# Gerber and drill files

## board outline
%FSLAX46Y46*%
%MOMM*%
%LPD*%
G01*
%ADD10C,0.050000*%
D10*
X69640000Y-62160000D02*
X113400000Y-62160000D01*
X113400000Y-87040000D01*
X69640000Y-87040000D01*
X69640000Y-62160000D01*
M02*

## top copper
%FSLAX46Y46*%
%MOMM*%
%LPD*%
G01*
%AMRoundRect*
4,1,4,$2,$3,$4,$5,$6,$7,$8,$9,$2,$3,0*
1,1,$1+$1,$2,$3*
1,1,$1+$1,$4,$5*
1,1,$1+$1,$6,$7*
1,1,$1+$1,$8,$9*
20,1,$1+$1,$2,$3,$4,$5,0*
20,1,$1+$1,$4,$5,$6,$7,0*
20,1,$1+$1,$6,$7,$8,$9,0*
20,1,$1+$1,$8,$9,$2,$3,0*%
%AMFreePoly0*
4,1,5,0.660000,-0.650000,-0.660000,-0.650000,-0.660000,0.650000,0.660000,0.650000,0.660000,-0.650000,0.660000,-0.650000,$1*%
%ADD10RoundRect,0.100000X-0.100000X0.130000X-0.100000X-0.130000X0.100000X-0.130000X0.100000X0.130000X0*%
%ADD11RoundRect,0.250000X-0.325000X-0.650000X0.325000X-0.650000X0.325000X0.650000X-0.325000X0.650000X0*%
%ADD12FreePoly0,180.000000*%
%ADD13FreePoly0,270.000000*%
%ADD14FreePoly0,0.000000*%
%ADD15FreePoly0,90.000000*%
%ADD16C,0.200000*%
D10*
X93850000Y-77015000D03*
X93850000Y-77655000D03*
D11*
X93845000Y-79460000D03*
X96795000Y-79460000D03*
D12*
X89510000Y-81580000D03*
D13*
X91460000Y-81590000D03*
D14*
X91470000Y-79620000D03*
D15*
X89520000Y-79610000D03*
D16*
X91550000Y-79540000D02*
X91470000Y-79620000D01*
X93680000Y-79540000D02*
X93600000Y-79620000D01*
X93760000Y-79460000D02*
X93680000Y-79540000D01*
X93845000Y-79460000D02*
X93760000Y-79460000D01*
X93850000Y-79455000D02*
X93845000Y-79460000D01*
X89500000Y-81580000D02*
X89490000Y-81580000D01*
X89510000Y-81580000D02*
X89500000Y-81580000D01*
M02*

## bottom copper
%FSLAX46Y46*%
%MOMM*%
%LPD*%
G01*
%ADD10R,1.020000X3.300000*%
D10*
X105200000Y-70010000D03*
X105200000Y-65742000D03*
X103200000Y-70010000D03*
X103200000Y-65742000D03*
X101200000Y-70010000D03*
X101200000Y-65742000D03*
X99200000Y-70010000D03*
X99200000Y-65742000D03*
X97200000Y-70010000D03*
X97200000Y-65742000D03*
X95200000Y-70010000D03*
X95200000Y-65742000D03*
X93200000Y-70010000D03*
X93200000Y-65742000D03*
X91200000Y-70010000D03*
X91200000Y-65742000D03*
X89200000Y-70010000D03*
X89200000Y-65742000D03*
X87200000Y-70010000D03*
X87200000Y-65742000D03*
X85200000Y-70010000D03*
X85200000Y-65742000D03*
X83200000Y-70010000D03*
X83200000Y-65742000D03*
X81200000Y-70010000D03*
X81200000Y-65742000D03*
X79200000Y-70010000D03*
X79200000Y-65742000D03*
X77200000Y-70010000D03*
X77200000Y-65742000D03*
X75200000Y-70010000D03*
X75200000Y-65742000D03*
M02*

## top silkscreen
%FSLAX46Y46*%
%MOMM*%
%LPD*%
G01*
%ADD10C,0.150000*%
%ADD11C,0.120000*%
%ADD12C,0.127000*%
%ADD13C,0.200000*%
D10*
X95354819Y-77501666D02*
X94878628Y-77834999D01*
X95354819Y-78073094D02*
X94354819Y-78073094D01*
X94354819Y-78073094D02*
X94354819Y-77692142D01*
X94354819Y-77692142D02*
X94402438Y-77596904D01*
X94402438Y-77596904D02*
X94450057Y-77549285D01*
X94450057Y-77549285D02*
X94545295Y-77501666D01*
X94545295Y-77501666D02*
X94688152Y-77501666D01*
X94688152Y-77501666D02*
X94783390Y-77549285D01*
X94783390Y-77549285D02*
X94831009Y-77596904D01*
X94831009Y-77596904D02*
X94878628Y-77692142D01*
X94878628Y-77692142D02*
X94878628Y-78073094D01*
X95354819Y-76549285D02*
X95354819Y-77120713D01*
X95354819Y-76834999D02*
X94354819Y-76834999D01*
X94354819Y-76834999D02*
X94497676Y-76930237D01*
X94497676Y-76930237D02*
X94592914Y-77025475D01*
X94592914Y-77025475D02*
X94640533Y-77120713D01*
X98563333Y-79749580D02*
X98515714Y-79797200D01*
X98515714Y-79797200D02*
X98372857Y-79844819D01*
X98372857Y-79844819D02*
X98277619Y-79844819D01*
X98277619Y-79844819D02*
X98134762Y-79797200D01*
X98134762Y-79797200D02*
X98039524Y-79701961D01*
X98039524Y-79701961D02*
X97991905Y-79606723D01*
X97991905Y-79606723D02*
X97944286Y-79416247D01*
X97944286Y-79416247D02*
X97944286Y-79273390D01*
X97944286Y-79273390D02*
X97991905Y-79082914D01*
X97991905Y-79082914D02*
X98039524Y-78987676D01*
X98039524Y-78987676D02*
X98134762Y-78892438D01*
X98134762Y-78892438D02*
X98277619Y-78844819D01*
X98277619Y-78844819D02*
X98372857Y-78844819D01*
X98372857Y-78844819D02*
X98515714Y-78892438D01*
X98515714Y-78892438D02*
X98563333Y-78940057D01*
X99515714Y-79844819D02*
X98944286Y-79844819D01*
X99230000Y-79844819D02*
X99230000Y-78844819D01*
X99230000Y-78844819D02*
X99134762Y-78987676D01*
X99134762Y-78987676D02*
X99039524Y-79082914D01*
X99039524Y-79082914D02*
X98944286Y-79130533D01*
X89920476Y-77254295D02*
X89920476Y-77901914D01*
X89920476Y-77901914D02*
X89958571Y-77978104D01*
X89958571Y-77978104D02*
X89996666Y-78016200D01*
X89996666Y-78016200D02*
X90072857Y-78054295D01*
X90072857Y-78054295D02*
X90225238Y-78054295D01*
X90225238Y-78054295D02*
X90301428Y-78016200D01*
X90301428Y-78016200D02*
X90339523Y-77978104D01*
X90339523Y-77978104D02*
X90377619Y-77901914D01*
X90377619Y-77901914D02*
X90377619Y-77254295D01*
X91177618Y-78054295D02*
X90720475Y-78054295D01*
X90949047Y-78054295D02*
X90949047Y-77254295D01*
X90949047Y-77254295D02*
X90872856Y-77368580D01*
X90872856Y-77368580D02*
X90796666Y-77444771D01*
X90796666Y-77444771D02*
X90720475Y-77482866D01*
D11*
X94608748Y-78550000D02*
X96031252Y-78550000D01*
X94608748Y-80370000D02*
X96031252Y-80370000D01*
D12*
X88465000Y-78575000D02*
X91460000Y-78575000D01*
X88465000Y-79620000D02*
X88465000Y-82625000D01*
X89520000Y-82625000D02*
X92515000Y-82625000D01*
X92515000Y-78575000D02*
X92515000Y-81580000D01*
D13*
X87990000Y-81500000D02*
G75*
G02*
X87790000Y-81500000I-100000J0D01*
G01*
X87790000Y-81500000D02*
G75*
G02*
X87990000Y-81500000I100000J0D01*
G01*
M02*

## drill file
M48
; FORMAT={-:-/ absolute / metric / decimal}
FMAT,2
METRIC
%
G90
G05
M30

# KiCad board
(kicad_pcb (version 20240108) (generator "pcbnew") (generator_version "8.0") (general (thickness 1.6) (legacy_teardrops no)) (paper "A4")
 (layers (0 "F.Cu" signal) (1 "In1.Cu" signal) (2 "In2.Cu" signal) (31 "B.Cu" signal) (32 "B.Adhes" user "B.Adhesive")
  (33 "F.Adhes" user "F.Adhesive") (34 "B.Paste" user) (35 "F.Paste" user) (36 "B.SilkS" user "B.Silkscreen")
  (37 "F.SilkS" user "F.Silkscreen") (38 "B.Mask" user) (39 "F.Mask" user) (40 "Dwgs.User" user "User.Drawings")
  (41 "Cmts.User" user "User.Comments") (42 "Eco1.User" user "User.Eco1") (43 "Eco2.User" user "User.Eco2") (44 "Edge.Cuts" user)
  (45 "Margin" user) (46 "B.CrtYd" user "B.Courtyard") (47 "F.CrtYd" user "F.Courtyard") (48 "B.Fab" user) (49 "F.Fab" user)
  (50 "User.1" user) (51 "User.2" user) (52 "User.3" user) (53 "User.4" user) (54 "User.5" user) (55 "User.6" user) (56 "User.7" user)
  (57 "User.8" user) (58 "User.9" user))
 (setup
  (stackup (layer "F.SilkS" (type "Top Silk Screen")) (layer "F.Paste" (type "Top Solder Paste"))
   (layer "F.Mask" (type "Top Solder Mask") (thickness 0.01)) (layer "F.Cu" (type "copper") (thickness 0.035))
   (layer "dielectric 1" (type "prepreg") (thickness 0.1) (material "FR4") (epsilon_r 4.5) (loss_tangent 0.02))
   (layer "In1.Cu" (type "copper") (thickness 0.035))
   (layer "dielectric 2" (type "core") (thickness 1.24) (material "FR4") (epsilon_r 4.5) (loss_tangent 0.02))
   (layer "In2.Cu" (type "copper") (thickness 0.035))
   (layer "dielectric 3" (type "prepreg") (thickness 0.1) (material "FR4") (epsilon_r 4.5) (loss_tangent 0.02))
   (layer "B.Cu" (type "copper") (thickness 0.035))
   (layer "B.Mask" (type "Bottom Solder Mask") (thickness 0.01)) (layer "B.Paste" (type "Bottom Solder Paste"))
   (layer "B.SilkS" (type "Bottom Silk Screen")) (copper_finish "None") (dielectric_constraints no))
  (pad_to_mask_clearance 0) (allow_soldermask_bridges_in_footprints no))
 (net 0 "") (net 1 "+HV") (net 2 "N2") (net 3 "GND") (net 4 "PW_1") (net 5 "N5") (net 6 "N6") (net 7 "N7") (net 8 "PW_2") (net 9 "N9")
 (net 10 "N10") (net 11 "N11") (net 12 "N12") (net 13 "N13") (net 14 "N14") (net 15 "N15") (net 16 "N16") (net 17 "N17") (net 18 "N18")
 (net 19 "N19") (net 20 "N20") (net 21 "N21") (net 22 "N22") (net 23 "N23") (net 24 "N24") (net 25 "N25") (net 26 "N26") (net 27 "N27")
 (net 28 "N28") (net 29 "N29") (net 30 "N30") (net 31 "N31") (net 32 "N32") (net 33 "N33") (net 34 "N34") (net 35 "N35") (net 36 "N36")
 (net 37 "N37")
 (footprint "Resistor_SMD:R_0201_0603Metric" (layer "F.Cu") (at 93.85 77.335 -90)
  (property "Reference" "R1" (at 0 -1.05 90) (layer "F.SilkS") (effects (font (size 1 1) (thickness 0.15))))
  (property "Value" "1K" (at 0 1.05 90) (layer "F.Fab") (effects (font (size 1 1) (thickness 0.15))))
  (pad "" smd roundrect (at -0.345 0 270) (size 0.318 0.36) (layers "F.Paste") (roundrect_rratio 0.25))
  (pad "" smd roundrect (at 0.345 0 270) (size 0.318 0.36) (layers "F.Paste") (roundrect_rratio 0.25))
  (pad "1" smd roundrect (at -0.32 0 270) (size 0.46 0.4) (layers "F.Cu" "F.Mask") (roundrect_rratio 0.25) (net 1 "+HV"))
  (pad "2" smd roundrect (at 0.32 0 270) (size 0.46 0.4) (layers "F.Cu" "F.Mask") (roundrect_rratio 0.25) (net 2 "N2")))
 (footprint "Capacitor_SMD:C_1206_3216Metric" (layer "F.Cu") (at 95.32 79.46)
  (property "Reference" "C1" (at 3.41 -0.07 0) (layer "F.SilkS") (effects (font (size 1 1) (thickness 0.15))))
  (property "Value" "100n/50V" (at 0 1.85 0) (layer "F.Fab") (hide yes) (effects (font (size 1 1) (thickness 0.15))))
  (fp_line (start -0.711252 -0.91) (end 0.711252 -0.91) (stroke (width 0.12) (type solid)) (layer "F.SilkS"))
  (fp_line (start -0.711252 0.91) (end 0.711252 0.91) (stroke (width 0.12) (type solid)) (layer "F.SilkS"))
  (pad "1" smd roundrect (at -1.475 0) (size 1.15 1.8) (layers "F.Cu" "F.Paste" "F.Mask") (roundrect_rratio 0.217391) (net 2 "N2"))
  (pad "2" smd roundrect (at 1.475 0) (size 1.15 1.8) (layers "F.Cu" "F.Paste" "F.Mask") (roundrect_rratio 0.217391) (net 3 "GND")))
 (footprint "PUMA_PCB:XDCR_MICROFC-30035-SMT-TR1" (layer "F.Cu") (at 90.49 80.6)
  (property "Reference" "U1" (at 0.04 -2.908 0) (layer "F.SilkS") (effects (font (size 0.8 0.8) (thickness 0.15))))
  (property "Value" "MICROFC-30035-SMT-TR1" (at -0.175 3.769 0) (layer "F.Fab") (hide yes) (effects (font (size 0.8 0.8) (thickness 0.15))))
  (fp_line (start -2.025 -2.025) (end 0.97 -2.025) (stroke (width 0.127) (type solid)) (layer "F.SilkS"))
  (fp_line (start -2.025 -0.98) (end -2.025 2.025) (stroke (width 0.127) (type solid)) (layer "F.SilkS"))
  (fp_line (start -0.97 2.025) (end 2.025 2.025) (stroke (width 0.127) (type solid)) (layer "F.SilkS"))
  (fp_line (start 2.025 -2.025) (end 2.025 0.98) (stroke (width 0.127) (type solid)) (layer "F.SilkS"))
  (fp_circle (center -2.6 0.9) (end -2.5 0.9) (stroke (width 0.2) (type solid)) (fill none) (layer "F.SilkS"))
  (pad "1" smd custom (at -0.98 0.98 180) (size 1.32 1.3) (layers "F.Cu") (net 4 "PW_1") (options (clearance outline) (anchor rect))
   (primitives))
  (pad "2" smd custom (at 0.97 0.99 270) (size 1.32 1.3) (layers "F.Cu") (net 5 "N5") (options (clearance outline) (anchor rect))
   (primitives))
  (pad "3" smd custom (at 0.98 -0.98) (size 1.32 1.3) (layers "F.Cu") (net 2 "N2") (options (clearance outline) (anchor rect)) (primitives)
   (teardrops (best_length_ratio 0.5) (max_length 1) (best_width_ratio 1) (max_width 2) (curve_points 5) (filter_ratio 0.9) (enabled yes)
    (allow_two_segments yes) (prefer_zone_connections yes)))
  (pad "4" smd custom (at -0.97 -0.99 90) (size 1.32 1.3) (layers "F.Cu") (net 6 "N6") (options (clearance outline) (anchor rect))
   (primitives)))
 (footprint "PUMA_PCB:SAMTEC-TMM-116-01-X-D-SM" (layer "B.Cu") (at 90.2 67.876 180)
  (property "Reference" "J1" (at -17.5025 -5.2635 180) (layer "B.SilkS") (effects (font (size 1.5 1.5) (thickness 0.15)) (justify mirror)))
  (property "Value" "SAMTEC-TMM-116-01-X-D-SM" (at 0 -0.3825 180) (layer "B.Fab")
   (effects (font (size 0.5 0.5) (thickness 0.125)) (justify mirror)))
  (pad "1" smd rect (at -15 -2.134 180) (size 1.02 3.3) (layers "B.Cu" "B.Paste") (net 4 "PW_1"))
  (pad "2" smd rect (at -15 2.134 180) (size 1.02 3.3) (layers "B.Cu" "B.Paste") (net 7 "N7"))
  (pad "3" smd rect (at -13 -2.134 180) (size 1.02 3.3) (layers "B.Cu" "B.Paste") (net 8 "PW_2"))
  (pad "4" smd rect (at -13 2.134 180) (size 1.02 3.3) (layers "B.Cu" "B.Paste") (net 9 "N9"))
  (pad "5" smd rect (at -11 -2.134 180) (size 1.02 3.3) (layers "B.Cu" "B.Paste") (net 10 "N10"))
  (pad "6" smd rect (at -11 2.134 180) (size 1.02 3.3) (layers "B.Cu" "B.Paste") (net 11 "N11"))
  (pad "7" smd rect (at -9 -2.134 180) (size 1.02 3.3) (layers "B.Cu" "B.Paste") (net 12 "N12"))
  (pad "8" smd rect (at -9 2.134 180) (size 1.02 3.3) (layers "B.Cu" "B.Paste") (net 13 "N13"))
  (pad "9" smd rect (at -7 -2.134 180) (size 1.02 3.3) (layers "B.Cu" "B.Paste") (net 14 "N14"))
  (pad "10" smd rect (at -7 2.134 180) (size 1.02 3.3) (layers "B.Cu" "B.Paste") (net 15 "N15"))
  (pad "11" smd rect (at -5 -2.134 180) (size 1.02 3.3) (layers "B.Cu" "B.Paste") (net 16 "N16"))
  (pad "12" smd rect (at -5 2.134 180) (size 1.02 3.3) (layers "B.Cu" "B.Paste") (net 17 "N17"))
  (pad "13" smd rect (at -3 -2.134 180) (size 1.02 3.3) (layers "B.Cu" "B.Paste") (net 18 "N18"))
  (pad "14" smd rect (at -3 2.134 180) (size 1.02 3.3) (layers "B.Cu" "B.Paste") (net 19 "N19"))
  (pad "15" smd rect (at -1 -2.134 180) (size 1.02 3.3) (layers "B.Cu" "B.Paste") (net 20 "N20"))
  (pad "16" smd rect (at -1 2.134 180) (size 1.02 3.3) (layers "B.Cu" "B.Paste") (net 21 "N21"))
  (pad "17" smd rect (at 1 -2.134 180) (size 1.02 3.3) (layers "B.Cu" "B.Paste") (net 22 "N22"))
  (pad "18" smd rect (at 1 2.134 180) (size 1.02 3.3) (layers "B.Cu" "B.Paste") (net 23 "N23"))
  (pad "19" smd rect (at 3 -2.134 180) (size 1.02 3.3) (layers "B.Cu" "B.Paste") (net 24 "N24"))
  (pad "20" smd rect (at 3 2.134 180) (size 1.02 3.3) (layers "B.Cu" "B.Paste") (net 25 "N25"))
  (pad "21" smd rect (at 5 -2.134 180) (size 1.02 3.3) (layers "B.Cu" "B.Paste") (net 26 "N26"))
  (pad "22" smd rect (at 5 2.134 180) (size 1.02 3.3) (layers "B.Cu" "B.Paste") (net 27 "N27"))
  (pad "23" smd rect (at 7 -2.134 180) (size 1.02 3.3) (layers "B.Cu" "B.Paste") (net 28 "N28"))
  (pad "24" smd rect (at 7 2.134 180) (size 1.02 3.3) (layers "B.Cu" "B.Paste") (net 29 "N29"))
  (pad "25" smd rect (at 9 -2.134 180) (size 1.02 3.3) (layers "B.Cu" "B.Paste") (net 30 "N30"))
  (pad "26" smd rect (at 9 2.134 180) (size 1.02 3.3) (layers "B.Cu" "B.Paste") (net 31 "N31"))
  (pad "27" smd rect (at 11 -2.134 180) (size 1.02 3.3) (layers "B.Cu" "B.Paste") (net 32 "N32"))
  (pad "28" smd rect (at 11 2.134 180) (size 1.02 3.3) (layers "B.Cu" "B.Paste") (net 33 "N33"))
  (pad "29" smd rect (at 13 -2.134 180) (size 1.02 3.3) (layers "B.Cu" "B.Paste") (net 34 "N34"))
  (pad "30" smd rect (at 13 2.134 180) (size 1.02 3.3) (layers "B.Cu" "B.Paste") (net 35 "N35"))
  (pad "31" smd rect (at 15 -2.134 180) (size 1.02 3.3) (layers "B.Cu" "B.Paste") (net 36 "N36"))
  (pad "32" smd rect (at 15 2.134 180) (size 1.02 3.3) (layers "B.Cu" "B.Paste") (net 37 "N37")))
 (gr_rect (start 69.64 62.16) (end 113.4 87.04) (stroke (width 0.05) (type default)) (fill none) (layer "Edge.Cuts"))
 (segment (start 91.55 79.54) (end 91.47 79.62) (width 0.2) (layer "F.Cu") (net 2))
 (segment (start 93.68 79.54) (end 93.6 79.62) (width 0.2) (layer "F.Cu") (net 2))
 (segment (start 93.76 79.46) (end 93.68 79.54) (width 0.2) (layer "F.Cu") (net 2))
 (segment (start 93.845 79.46) (end 93.76 79.46) (width 0.2) (layer "F.Cu") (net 2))
 (segment (start 93.85 79.455) (end 93.845 79.46) (width 0.2) (layer "F.Cu") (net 2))
 (segment (start 89.5 81.58) (end 89.49 81.58) (width 0.2) (layer "F.Cu") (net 4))
 (segment (start 89.51 81.58) (end 89.5 81.58) (width 0.2) (layer "F.Cu") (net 4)))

